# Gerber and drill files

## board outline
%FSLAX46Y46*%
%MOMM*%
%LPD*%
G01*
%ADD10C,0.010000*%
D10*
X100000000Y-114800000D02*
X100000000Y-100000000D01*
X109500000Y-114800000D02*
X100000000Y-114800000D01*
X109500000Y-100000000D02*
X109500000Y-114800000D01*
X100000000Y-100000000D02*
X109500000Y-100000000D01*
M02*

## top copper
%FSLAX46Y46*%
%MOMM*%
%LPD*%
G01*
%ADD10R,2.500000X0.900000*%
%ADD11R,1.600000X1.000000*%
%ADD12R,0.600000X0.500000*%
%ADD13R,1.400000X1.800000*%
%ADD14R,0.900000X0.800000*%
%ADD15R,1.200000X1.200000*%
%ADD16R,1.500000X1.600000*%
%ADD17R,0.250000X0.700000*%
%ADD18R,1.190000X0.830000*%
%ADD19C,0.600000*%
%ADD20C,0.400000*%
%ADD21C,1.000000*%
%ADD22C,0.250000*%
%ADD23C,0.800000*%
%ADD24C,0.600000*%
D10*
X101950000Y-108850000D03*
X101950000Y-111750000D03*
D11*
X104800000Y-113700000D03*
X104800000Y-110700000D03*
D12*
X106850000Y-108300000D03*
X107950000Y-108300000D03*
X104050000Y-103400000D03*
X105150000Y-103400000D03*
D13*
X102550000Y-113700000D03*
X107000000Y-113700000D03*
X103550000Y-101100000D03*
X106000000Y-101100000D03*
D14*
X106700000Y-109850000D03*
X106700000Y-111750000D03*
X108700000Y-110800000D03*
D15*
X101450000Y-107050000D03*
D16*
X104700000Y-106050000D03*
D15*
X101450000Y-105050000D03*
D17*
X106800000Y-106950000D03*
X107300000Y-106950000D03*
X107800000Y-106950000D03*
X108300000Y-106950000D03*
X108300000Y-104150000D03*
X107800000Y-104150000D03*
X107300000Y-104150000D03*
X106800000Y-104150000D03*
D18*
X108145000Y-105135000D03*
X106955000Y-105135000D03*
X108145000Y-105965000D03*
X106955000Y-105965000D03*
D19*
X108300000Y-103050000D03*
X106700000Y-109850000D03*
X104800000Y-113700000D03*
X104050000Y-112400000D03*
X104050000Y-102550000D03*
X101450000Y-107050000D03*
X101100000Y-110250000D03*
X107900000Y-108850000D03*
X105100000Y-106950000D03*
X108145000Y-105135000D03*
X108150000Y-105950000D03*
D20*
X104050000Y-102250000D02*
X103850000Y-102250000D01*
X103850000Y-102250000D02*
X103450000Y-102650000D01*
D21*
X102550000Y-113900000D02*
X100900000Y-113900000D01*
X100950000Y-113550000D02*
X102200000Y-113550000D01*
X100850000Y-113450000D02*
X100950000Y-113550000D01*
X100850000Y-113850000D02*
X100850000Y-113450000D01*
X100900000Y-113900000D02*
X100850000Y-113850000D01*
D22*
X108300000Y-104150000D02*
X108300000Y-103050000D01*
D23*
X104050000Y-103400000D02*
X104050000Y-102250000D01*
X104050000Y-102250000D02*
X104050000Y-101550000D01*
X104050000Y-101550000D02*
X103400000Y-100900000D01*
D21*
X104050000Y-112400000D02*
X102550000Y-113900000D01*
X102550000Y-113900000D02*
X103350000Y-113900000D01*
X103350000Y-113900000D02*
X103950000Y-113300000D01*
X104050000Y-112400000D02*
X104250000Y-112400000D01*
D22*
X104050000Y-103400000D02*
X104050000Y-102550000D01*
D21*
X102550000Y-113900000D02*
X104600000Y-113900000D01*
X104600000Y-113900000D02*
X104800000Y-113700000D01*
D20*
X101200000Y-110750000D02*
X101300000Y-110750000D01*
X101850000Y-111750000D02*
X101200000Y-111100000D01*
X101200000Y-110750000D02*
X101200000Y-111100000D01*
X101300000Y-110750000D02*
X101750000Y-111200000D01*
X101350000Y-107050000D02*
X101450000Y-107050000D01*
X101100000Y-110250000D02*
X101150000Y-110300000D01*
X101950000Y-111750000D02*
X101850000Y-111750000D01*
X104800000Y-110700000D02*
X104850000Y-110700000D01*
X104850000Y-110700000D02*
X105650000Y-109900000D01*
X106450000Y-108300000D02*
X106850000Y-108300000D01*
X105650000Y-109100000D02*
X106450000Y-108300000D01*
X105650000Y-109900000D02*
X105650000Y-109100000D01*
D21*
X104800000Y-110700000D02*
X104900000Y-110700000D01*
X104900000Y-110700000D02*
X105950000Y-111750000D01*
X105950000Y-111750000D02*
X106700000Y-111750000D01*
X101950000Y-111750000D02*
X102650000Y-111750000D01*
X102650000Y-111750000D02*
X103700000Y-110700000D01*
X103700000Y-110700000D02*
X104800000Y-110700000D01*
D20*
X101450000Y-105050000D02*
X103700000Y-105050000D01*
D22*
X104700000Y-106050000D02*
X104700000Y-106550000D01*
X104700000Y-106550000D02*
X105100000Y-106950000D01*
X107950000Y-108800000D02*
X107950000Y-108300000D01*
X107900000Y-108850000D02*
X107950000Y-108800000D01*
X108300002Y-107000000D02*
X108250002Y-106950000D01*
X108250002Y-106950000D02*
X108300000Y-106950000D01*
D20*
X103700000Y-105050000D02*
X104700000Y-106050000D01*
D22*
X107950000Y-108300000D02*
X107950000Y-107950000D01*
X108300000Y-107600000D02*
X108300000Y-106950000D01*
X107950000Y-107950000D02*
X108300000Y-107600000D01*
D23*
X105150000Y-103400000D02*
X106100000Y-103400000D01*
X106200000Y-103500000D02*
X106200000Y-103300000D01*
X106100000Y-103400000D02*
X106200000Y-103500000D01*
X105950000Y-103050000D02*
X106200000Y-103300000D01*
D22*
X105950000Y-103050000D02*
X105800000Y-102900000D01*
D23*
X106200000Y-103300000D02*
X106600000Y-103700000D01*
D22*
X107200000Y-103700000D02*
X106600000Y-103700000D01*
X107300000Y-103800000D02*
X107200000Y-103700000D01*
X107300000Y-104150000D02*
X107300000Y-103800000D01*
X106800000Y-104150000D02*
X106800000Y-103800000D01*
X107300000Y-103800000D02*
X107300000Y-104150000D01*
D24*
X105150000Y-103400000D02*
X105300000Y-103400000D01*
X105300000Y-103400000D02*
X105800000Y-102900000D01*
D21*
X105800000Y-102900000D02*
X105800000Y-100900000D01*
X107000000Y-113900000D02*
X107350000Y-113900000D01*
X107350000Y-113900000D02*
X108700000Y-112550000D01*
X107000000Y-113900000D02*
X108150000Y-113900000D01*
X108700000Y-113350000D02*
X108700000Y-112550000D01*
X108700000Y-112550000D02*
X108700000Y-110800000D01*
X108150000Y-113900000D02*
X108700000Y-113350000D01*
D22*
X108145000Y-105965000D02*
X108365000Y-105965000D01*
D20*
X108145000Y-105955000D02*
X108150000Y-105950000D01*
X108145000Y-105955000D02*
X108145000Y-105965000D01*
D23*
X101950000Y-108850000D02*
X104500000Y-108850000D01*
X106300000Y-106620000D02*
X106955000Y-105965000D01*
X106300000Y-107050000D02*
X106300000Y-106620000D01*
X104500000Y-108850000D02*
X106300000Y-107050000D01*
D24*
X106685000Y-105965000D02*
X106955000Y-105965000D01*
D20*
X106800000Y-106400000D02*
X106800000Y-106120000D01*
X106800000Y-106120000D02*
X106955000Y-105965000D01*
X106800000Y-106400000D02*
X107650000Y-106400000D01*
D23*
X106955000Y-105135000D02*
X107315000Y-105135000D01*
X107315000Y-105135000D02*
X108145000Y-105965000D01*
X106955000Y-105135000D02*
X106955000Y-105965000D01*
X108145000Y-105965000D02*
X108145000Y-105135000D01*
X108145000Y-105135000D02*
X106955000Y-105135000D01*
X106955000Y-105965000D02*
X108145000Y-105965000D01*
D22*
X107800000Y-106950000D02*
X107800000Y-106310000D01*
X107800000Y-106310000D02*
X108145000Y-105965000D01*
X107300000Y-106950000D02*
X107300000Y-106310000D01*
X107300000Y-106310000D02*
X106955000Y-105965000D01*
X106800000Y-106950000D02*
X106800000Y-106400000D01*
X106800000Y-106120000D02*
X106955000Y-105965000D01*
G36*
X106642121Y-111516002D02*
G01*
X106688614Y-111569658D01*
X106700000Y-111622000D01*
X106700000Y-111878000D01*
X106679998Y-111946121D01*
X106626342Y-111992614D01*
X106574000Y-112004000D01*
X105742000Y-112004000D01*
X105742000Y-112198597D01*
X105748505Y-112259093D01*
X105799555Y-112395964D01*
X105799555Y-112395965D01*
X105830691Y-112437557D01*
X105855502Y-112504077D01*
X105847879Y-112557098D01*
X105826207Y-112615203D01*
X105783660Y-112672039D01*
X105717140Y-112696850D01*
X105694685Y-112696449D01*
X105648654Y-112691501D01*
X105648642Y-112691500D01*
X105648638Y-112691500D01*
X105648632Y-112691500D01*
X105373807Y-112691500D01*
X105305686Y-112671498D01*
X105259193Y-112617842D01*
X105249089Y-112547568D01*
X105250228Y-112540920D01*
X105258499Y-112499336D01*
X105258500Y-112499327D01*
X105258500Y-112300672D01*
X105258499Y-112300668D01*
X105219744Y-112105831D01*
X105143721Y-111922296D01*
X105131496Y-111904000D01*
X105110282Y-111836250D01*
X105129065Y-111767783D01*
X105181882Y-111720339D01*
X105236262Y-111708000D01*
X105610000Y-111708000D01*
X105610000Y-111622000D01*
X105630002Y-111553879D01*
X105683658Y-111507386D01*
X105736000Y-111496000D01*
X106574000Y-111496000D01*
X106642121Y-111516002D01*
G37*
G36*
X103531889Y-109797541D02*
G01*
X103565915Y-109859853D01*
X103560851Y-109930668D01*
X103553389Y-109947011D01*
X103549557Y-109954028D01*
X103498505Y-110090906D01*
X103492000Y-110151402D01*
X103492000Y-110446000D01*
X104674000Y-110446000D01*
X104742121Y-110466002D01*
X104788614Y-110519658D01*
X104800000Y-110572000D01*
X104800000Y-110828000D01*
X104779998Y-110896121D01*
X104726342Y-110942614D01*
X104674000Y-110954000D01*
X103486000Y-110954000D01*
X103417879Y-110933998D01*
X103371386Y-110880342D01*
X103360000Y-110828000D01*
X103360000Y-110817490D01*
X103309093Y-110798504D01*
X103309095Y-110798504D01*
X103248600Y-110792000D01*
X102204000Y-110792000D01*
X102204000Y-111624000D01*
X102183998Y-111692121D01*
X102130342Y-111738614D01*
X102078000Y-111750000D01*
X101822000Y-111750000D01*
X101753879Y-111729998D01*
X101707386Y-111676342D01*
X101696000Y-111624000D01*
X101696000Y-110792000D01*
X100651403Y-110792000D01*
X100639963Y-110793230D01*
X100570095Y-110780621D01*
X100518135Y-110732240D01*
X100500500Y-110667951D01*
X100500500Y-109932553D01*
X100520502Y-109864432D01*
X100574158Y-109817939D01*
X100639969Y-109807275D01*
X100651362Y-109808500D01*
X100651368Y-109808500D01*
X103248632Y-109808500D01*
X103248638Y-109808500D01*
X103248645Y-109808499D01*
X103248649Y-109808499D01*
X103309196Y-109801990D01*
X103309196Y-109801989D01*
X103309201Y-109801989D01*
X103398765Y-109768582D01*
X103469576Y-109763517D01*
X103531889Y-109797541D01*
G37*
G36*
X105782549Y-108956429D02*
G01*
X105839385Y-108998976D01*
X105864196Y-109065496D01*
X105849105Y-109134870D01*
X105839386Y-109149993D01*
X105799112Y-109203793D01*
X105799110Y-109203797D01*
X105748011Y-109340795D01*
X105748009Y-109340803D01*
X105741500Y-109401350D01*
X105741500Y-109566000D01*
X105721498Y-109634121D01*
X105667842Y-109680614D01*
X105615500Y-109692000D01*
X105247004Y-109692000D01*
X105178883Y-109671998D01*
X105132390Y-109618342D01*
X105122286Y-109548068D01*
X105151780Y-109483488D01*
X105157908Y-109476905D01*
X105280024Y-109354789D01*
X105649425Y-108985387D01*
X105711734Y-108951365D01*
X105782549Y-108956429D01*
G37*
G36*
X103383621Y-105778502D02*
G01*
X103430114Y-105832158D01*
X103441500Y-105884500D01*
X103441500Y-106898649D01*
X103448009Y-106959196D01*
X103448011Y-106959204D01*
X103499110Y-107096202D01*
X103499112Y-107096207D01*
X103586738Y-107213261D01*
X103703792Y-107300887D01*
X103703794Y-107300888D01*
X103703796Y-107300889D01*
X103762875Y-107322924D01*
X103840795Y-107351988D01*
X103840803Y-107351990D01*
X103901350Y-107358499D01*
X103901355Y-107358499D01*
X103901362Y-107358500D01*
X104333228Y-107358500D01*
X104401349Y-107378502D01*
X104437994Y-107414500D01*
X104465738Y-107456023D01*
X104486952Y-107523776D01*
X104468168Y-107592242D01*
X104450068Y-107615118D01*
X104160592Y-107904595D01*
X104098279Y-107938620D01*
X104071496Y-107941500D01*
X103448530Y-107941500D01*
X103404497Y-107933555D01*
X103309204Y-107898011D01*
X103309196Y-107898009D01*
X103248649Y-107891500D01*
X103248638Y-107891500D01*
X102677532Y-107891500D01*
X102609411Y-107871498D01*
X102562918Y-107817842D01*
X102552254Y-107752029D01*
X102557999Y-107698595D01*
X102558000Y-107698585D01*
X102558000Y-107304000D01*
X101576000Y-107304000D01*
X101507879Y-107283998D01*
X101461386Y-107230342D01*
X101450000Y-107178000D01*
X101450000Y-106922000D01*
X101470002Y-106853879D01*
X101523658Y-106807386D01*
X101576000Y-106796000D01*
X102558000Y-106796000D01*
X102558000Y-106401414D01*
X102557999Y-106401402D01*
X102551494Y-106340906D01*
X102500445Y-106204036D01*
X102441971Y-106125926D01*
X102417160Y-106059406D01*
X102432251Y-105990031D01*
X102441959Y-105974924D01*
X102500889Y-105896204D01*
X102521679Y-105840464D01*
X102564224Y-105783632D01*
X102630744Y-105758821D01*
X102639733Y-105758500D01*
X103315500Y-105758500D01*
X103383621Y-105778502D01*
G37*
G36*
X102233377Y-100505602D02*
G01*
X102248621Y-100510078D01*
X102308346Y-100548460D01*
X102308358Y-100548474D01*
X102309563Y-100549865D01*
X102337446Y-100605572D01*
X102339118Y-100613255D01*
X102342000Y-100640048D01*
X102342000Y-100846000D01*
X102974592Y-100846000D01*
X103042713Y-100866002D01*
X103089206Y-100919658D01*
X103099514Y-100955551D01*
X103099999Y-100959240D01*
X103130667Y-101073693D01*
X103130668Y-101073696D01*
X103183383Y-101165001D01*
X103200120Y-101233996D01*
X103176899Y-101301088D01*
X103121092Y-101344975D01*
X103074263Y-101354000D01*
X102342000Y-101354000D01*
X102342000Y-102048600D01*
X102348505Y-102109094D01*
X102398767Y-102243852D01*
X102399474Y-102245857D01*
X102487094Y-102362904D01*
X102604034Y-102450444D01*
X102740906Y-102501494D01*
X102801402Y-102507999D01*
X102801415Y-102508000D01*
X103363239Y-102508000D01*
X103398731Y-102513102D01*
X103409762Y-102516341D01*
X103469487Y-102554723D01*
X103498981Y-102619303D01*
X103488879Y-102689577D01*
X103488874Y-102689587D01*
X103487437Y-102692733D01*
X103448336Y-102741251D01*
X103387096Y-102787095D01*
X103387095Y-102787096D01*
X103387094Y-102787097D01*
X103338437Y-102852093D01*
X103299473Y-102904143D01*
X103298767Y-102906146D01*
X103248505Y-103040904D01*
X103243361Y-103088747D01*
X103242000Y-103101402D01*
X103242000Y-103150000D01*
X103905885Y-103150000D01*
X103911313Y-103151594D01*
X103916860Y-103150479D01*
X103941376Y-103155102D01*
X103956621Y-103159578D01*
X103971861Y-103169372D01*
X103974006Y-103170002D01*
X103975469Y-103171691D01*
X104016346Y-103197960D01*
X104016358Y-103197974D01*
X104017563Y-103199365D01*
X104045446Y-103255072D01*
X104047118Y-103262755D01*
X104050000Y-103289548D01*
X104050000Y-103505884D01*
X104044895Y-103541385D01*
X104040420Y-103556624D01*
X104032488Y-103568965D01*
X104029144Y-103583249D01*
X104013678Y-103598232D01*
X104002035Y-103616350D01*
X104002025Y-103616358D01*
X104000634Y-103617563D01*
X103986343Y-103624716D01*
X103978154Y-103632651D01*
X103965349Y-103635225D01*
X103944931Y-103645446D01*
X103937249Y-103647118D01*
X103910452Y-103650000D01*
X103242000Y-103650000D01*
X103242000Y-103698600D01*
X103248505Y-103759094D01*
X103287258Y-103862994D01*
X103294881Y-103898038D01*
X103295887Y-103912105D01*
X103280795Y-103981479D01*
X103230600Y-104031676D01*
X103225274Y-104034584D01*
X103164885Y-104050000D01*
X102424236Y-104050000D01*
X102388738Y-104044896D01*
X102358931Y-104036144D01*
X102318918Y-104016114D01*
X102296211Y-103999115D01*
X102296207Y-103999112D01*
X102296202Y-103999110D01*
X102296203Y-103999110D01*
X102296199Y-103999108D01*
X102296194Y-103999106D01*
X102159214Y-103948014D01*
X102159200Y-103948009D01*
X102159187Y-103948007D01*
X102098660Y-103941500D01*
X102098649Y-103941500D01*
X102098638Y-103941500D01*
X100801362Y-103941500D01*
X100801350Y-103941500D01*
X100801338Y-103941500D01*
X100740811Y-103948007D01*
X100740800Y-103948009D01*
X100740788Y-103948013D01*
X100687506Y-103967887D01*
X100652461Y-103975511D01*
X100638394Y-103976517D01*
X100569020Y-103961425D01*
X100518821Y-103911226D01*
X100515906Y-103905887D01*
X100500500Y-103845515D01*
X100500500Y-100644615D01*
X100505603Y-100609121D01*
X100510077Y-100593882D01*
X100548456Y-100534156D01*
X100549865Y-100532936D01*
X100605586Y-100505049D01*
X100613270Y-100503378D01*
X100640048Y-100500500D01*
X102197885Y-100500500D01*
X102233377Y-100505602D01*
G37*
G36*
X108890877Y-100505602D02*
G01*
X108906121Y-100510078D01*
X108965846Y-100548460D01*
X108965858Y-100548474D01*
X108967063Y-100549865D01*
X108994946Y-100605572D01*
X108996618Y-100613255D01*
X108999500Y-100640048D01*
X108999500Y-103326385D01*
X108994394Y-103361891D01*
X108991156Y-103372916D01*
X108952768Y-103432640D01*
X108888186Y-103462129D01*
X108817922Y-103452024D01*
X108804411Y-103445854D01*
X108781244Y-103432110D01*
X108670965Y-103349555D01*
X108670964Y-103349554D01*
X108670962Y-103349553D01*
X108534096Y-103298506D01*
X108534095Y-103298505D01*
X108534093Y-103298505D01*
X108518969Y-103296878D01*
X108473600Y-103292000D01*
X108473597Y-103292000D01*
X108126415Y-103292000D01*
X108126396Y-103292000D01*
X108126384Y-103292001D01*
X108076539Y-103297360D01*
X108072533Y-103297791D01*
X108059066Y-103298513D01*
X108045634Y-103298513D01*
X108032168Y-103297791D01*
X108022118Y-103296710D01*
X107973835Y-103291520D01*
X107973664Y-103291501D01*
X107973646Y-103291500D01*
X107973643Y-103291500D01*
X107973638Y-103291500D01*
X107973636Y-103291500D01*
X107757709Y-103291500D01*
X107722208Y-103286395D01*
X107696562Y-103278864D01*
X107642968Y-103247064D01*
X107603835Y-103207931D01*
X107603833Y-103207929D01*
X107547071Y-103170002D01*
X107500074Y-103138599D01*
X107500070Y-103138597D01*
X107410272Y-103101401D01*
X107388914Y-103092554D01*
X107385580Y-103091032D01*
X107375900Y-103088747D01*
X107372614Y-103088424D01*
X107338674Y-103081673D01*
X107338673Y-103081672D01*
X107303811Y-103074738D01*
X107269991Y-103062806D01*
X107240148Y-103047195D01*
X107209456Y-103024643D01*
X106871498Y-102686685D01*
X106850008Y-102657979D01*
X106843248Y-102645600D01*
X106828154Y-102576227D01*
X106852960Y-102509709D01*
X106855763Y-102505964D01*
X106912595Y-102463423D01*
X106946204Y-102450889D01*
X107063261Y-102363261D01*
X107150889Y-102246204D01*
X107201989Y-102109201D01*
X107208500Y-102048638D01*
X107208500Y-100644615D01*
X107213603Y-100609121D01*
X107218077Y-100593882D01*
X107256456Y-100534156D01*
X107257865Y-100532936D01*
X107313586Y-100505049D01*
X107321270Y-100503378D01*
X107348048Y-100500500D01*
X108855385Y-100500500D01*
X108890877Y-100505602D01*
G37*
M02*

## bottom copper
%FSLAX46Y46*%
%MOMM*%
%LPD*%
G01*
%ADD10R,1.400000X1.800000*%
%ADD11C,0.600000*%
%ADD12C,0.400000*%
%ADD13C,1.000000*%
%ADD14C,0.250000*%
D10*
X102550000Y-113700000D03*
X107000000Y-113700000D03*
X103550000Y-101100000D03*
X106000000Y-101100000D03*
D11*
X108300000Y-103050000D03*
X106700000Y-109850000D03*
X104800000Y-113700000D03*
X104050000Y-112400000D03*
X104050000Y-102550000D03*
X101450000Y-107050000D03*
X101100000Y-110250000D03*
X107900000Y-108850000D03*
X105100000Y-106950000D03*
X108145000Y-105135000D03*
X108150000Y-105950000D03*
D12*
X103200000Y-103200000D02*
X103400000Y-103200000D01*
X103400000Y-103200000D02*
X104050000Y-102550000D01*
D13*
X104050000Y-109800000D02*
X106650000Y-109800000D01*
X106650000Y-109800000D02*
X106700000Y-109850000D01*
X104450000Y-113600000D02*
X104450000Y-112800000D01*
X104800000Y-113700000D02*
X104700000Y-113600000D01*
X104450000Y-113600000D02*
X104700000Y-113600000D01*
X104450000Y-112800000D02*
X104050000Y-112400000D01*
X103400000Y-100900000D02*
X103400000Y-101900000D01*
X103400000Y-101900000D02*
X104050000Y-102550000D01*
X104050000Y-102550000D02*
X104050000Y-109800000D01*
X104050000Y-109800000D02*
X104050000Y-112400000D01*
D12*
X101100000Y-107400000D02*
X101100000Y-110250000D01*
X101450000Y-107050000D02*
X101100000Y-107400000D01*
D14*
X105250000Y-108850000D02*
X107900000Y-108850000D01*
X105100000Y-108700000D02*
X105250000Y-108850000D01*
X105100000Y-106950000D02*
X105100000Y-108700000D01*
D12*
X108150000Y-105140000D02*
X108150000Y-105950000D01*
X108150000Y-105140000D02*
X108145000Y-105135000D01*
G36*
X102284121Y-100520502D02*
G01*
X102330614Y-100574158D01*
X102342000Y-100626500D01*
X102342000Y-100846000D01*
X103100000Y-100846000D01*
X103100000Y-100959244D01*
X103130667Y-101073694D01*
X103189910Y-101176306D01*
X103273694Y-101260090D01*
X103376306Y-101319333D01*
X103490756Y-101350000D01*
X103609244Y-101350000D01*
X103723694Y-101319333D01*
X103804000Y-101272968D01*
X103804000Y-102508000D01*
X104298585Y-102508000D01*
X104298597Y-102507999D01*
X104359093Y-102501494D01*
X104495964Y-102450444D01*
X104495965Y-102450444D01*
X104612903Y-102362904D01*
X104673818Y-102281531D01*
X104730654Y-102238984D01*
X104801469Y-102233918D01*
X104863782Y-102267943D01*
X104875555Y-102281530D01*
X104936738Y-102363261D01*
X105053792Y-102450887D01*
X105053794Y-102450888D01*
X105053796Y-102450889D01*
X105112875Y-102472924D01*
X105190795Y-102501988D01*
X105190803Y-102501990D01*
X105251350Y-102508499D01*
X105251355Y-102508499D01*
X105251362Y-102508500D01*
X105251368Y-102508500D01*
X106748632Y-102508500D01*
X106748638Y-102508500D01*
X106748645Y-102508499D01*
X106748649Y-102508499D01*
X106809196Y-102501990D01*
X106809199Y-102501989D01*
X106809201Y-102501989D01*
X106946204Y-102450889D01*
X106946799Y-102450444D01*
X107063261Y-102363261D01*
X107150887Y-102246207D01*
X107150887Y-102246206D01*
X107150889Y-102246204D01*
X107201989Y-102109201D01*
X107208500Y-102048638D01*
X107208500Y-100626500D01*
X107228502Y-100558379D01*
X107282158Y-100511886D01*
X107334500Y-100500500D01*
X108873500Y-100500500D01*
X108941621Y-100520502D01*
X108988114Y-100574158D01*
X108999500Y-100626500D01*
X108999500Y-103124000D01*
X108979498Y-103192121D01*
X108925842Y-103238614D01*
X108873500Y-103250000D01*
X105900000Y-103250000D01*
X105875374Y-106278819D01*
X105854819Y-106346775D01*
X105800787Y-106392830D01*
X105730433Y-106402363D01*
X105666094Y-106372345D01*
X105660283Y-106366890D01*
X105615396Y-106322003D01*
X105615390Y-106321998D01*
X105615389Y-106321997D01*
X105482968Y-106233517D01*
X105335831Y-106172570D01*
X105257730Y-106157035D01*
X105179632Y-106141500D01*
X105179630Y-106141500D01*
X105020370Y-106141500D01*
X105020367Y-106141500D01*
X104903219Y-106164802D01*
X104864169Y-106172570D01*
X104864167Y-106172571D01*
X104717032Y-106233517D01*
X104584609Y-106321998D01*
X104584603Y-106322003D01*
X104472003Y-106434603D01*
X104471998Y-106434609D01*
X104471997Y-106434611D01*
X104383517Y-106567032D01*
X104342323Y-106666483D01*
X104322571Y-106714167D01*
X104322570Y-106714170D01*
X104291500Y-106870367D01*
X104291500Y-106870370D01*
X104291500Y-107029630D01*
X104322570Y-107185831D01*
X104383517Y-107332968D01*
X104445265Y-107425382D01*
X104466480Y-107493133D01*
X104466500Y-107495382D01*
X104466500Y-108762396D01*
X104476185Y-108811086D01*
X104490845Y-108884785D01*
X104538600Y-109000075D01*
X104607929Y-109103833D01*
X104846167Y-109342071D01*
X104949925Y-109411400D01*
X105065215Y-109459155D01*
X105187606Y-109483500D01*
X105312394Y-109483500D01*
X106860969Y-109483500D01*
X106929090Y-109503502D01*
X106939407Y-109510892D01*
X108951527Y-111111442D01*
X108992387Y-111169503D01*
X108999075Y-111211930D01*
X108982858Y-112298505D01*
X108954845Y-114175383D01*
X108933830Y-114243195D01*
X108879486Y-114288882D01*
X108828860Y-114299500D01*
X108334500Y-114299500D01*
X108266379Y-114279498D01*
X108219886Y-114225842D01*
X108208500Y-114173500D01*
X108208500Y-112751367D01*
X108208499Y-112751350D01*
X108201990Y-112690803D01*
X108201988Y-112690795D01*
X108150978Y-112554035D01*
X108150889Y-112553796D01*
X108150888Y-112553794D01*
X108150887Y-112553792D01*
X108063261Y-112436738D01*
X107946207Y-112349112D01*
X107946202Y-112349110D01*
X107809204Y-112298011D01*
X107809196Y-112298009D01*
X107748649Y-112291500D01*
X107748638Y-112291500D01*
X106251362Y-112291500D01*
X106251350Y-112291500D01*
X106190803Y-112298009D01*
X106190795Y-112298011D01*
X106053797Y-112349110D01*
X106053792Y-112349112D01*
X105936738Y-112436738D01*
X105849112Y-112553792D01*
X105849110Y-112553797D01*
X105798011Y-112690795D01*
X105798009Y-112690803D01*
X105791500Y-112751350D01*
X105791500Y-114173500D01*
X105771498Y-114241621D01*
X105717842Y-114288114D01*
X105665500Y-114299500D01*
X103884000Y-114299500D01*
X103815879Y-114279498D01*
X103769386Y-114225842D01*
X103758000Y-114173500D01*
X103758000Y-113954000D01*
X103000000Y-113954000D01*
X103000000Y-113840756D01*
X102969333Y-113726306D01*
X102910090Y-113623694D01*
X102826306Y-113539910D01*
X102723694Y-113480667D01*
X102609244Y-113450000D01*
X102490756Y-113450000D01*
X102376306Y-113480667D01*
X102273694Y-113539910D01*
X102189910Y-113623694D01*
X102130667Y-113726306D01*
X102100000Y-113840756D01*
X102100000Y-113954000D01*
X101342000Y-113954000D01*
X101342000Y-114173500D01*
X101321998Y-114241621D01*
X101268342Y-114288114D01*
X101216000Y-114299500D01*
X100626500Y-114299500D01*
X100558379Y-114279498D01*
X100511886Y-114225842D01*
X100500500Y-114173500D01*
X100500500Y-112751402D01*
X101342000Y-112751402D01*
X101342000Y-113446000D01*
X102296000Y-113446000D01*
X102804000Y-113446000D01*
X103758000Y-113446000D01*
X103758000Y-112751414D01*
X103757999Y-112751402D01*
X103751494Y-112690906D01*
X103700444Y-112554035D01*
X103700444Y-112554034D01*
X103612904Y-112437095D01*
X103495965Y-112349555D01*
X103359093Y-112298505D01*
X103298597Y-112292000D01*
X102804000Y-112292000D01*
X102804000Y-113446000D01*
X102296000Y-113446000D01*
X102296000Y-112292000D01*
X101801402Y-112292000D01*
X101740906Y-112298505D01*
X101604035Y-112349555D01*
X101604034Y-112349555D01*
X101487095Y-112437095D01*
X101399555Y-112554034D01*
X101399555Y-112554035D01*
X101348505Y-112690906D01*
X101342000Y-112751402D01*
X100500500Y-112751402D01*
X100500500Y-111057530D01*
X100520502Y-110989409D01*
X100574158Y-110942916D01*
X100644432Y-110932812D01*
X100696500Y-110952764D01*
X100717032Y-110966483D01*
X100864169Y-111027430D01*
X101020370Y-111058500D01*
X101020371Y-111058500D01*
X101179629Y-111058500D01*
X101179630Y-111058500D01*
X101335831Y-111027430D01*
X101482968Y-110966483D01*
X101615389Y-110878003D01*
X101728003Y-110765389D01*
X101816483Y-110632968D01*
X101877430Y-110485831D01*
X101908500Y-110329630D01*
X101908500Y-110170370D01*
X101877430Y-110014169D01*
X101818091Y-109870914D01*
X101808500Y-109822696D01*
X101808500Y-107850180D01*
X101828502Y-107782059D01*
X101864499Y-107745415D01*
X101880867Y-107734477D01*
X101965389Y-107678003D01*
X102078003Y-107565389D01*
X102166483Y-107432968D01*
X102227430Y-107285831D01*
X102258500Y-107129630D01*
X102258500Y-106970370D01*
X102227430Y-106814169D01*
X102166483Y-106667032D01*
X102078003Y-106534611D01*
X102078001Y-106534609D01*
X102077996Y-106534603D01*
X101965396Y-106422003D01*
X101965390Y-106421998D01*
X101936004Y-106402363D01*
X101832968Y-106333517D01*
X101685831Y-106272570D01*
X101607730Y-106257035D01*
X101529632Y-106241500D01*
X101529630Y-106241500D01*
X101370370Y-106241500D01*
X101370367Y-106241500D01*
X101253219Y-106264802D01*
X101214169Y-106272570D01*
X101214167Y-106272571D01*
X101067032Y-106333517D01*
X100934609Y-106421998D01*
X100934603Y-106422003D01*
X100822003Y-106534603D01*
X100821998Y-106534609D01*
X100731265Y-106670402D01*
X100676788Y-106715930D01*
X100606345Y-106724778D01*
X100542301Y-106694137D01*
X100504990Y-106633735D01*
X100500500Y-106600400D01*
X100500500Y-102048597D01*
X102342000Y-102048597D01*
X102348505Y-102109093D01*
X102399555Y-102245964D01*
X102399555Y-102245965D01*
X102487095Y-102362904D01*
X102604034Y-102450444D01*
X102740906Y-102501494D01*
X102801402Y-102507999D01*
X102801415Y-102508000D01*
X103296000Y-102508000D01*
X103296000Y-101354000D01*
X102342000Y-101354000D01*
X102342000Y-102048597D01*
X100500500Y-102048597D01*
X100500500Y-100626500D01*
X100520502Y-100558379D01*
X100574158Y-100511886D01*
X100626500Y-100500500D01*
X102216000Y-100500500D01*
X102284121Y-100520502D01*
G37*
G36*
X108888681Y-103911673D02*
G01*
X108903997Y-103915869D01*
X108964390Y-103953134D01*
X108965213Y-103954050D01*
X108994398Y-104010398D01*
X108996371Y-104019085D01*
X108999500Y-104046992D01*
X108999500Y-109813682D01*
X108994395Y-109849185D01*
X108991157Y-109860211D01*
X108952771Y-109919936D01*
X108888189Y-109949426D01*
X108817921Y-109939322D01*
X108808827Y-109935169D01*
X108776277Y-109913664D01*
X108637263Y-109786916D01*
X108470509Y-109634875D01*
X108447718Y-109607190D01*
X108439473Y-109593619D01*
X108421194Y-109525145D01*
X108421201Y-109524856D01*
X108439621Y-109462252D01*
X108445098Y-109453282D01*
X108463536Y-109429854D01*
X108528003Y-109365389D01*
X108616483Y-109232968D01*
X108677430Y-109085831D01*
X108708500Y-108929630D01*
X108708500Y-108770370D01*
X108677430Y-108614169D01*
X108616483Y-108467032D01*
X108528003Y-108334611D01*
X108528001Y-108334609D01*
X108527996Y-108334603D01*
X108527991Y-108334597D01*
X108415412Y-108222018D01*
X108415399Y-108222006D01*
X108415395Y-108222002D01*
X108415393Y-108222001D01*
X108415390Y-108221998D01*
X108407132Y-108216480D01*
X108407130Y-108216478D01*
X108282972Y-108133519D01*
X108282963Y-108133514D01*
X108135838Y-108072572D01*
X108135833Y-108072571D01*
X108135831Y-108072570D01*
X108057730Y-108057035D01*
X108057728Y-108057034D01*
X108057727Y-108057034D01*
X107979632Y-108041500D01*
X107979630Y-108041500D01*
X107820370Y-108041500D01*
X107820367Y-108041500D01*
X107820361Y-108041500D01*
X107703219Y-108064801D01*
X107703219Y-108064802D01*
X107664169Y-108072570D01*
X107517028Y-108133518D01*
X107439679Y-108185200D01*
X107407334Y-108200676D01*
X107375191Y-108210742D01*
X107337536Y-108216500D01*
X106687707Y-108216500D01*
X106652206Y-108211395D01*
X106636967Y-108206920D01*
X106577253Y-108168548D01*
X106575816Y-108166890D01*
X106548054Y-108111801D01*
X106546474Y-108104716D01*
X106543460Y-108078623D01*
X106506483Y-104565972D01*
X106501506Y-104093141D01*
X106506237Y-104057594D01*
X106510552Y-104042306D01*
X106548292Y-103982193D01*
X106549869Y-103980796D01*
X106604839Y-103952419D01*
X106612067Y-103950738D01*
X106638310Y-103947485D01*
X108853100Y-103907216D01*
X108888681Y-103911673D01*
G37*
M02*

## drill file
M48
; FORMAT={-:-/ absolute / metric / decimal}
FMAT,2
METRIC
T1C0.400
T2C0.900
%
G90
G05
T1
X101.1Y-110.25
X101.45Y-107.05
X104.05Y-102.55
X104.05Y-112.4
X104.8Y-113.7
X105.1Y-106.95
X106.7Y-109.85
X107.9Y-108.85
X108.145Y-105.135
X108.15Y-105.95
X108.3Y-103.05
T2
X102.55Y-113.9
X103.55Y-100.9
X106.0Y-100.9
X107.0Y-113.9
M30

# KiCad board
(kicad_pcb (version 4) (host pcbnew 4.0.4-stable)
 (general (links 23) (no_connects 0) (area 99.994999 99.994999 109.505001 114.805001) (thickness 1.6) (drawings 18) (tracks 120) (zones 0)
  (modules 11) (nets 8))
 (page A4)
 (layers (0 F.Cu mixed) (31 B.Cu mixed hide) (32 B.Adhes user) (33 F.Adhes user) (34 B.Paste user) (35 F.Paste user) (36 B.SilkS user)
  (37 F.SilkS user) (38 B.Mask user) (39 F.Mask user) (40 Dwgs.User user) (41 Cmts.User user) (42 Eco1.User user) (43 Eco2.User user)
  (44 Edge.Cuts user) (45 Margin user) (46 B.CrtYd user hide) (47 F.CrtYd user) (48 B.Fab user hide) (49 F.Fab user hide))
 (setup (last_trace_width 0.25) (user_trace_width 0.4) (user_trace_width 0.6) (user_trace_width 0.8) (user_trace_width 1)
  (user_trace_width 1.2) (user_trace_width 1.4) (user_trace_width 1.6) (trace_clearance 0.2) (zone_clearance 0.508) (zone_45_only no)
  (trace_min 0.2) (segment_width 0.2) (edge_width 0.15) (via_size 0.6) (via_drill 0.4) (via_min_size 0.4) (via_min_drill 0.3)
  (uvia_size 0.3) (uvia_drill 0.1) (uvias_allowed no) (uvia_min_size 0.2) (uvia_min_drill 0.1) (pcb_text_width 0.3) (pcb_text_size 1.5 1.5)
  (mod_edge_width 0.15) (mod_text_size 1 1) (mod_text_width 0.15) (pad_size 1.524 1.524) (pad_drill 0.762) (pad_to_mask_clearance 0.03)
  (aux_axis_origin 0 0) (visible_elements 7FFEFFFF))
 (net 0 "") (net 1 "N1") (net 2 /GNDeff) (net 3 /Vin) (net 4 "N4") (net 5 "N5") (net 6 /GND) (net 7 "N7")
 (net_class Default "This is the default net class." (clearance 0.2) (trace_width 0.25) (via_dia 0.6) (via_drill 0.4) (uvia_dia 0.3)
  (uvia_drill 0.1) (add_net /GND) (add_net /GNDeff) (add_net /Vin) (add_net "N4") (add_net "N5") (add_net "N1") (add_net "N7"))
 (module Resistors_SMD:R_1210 (layer F.Cu) (at 101.95 110.3 270)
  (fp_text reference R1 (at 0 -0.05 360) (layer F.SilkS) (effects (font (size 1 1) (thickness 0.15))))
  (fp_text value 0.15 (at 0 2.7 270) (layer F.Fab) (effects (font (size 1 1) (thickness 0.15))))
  (pad 1 smd rect (at -1.45 0 270) (size 0.9 2.5) (layers F.Cu F.Paste F.Mask) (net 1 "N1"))
  (pad 2 smd rect (at 1.45 0 270) (size 0.9 2.5) (layers F.Cu F.Paste F.Mask) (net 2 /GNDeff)))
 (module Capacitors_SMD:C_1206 (layer F.Cu) (at 104.8 112.2 90)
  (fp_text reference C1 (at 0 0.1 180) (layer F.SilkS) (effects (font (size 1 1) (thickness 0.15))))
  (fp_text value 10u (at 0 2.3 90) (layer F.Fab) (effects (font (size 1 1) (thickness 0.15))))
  (pad 1 smd rect (at -1.5 0 90) (size 1 1.6) (layers F.Cu F.Paste F.Mask) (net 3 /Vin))
  (pad 2 smd rect (at 1.5 0 90) (size 1 1.6) (layers F.Cu F.Paste F.Mask) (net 2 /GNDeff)))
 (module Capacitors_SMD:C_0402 (layer F.Cu) (at 107.4 108.3)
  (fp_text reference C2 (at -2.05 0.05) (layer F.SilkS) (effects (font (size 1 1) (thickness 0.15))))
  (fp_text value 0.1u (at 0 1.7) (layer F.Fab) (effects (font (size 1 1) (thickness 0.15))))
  (pad 1 smd rect (at -0.55 0) (size 0.6 0.5) (layers F.Cu F.Paste F.Mask) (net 2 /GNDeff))
  (pad 2 smd rect (at 0.55 0) (size 0.6 0.5) (layers F.Cu F.Paste F.Mask) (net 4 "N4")))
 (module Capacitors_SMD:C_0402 (layer F.Cu) (at 104.6 103.4)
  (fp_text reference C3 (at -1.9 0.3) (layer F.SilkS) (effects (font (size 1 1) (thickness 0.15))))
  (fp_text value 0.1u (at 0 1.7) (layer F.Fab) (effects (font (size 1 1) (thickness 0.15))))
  (pad 1 smd rect (at -0.55 0) (size 0.6 0.5) (layers F.Cu F.Paste F.Mask) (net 3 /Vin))
  (pad 2 smd rect (at 0.55 0) (size 0.6 0.5) (layers F.Cu F.Paste F.Mask) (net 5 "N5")))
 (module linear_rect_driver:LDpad (layer F.Cu) (at 103 113.85 270)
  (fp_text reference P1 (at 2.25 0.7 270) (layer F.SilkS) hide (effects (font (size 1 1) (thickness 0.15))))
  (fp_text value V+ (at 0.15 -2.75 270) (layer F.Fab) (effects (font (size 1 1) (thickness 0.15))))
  (pad 1 thru_hole rect (at 0.05 0.45 270) (size 1.8 1.4) (drill 0.9 (offset -0.2 0)) (layers *.Cu *.Mask) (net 3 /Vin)))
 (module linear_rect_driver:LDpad (layer F.Cu) (at 107.45 113.85 270)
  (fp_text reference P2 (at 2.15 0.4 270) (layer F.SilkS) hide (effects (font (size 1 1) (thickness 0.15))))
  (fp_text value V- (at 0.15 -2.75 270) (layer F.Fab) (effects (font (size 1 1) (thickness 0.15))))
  (pad 1 thru_hole rect (at 0.05 0.45 270) (size 1.8 1.4) (drill 0.9 (offset -0.2 0)) (layers *.Cu *.Mask) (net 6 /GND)))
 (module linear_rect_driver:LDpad (layer F.Cu) (at 103.1 100.95 90)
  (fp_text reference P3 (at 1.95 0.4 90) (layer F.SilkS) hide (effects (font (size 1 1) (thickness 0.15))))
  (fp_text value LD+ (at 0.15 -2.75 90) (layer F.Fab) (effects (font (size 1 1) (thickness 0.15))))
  (pad 1 thru_hole rect (at 0.05 0.45 90) (size 1.8 1.4) (drill 0.9 (offset -0.2 0)) (layers *.Cu *.Mask) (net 3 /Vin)))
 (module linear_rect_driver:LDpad (layer F.Cu) (at 105.55 100.95 90)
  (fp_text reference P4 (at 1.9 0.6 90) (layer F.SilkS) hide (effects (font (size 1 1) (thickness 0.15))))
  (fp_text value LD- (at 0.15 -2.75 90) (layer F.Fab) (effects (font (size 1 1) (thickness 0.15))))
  (pad 1 thru_hole rect (at 0.05 0.45 90) (size 1.8 1.4) (drill 0.9 (offset -0.2 0)) (layers *.Cu *.Mask) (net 5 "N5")))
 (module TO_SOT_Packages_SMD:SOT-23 (layer F.Cu) (at 107.7 110.8)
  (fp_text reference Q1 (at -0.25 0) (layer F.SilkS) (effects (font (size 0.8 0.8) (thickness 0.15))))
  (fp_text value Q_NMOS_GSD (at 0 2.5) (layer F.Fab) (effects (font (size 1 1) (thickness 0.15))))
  (pad 1 smd rect (at -1 -0.95) (size 0.9 0.8) (layers F.Cu F.Paste F.Mask) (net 3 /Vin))
  (pad 2 smd rect (at -1 0.95) (size 0.9 0.8) (layers F.Cu F.Paste F.Mask) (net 2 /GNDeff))
  (pad 3 smd rect (at 1 0) (size 0.9 0.8) (layers F.Cu F.Paste F.Mask) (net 6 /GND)))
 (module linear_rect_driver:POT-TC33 (layer F.Cu) (at 103.95 106.05 270)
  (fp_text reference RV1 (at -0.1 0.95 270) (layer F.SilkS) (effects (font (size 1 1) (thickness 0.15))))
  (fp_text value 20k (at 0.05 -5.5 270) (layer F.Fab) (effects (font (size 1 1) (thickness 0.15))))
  (pad 3 smd rect (at 1 2.5 270) (size 1.2 1.2) (layers F.Cu F.Paste F.Mask) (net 2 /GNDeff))
  (pad 2 smd rect (at 0 -0.75 270) (size 1.6 1.5) (layers F.Cu F.Paste F.Mask) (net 4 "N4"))
  (pad 1 smd rect (at -1 2.5 270) (size 1.2 1.2) (layers F.Cu F.Paste F.Mask) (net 4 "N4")))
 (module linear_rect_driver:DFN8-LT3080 (layer F.Cu) (at 107.55 105.55 90)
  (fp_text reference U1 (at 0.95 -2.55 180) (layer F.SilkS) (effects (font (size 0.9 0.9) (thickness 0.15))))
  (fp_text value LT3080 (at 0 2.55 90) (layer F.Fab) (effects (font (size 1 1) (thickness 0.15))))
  (pad 1 smd rect (at -1.4 -0.75 90) (size 0.7 0.25) (layers F.Cu F.Paste F.Mask) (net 1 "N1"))
  (pad 1 smd rect (at -1.4 -0.25 90) (size 0.7 0.25) (layers F.Cu F.Paste F.Mask) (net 1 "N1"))
  (pad 1 smd rect (at -1.4 0.25 90) (size 0.7 0.25) (layers F.Cu F.Paste F.Mask) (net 1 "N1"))
  (pad 2 smd rect (at -1.4 0.75 90) (size 0.7 0.25) (layers F.Cu F.Paste F.Mask) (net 4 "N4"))
  (pad 3 smd rect (at 1.4 0.75 90) (size 0.7 0.25) (layers F.Cu F.Paste F.Mask) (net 3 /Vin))
  (pad 5 smd rect (at 1.4 0.25 90) (size 0.7 0.25) (layers F.Cu F.Paste F.Mask) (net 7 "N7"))
  (pad 4 smd rect (at 1.4 -0.25 90) (size 0.7 0.25) (layers F.Cu F.Paste F.Mask) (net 5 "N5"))
  (pad 4 smd rect (at 1.4 -0.75 90) (size 0.7 0.25) (layers F.Cu F.Paste F.Mask) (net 5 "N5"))
  (pad 1 smd rect (at 0.415 0.595 90) (size 0.83 1.19) (layers F.Cu F.Paste F.Mask) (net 1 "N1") (solder_paste_margin_ratio -0.2))
  (pad 1 smd rect (at 0.415 -0.595 90) (size 0.83 1.19) (layers F.Cu F.Paste F.Mask) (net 1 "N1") (solder_paste_margin_ratio -0.2))
  (pad 1 smd rect (at -0.415 0.595 90) (size 0.83 1.19) (layers F.Cu F.Paste F.Mask) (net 1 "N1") (solder_paste_margin_ratio -0.2))
  (pad 1 smd rect (at -0.415 -0.595 90) (size 0.83 1.19) (layers F.Cu F.Paste F.Mask) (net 1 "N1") (solder_paste_margin_ratio -0.2)))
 (gr_line (start 100 114.8) (end 100 100) (angle 90) (layer Edge.Cuts) (width 0.01))
 (gr_line (start 109.5 114.8) (end 100 114.8) (angle 90) (layer Edge.Cuts) (width 0.01))
 (gr_line (start 109.5 100) (end 109.5 114.8) (angle 90) (layer Edge.Cuts) (width 0.01))
 (gr_line (start 100 100) (end 109.5 100) (angle 90) (layer Edge.Cuts) (width 0.01))
 (segment (start 104.05 102.25) (end 103.85 102.25) (width 0.4) (layer F.Cu) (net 3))
 (segment (start 103.85 102.25) (end 103.45 102.65) (width 0.4) (layer F.Cu) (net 3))
 (segment (start 103.2 103.2) (end 103.4 103.2) (width 0.4) (layer B.Cu) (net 3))
 (segment (start 103.4 103.2) (end 104.05 102.55) (width 0.4) (layer B.Cu) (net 3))
 (segment (start 102.55 113.9) (end 100.9 113.9) (width 1) (layer F.Cu) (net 3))
 (segment (start 100.95 113.55) (end 102.2 113.55) (width 1) (layer F.Cu) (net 3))
 (segment (start 100.85 113.45) (end 100.95 113.55) (width 1) (layer F.Cu) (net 3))
 (segment (start 100.85 113.85) (end 100.85 113.45) (width 1) (layer F.Cu) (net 3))
 (segment (start 100.9 113.9) (end 100.85 113.85) (width 1) (layer F.Cu) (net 3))
 (segment (start 108.3 104.15) (end 108.3 103.05) (width 0.25) (layer F.Cu) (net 3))
 (via (at 108.3 103.05) (size 0.6) (drill 0.4) (layers F.Cu B.Cu) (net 3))
 (segment (start 104.05 103.4) (end 104.05 102.25) (width 0.8) (layer F.Cu) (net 3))
 (segment (start 104.05 102.25) (end 104.05 101.55) (width 0.8) (layer F.Cu) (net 3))
 (segment (start 104.05 101.55) (end 103.4 100.9) (width 0.8) (layer F.Cu) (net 3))
 (via (at 106.7 109.85) (size 0.6) (drill 0.4) (layers F.Cu B.Cu) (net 3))
 (segment (start 104.05 109.8) (end 106.65 109.8) (width 1) (layer B.Cu) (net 3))
 (segment (start 106.65 109.8) (end 106.7 109.85) (width 1) (layer B.Cu) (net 3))
 (segment (start 104.45 113.6) (end 104.45 112.8) (width 1) (layer B.Cu) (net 3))
 (segment (start 104.8 113.7) (end 104.7 113.6) (width 1) (layer B.Cu) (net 3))
 (segment (start 104.45 113.6) (end 104.7 113.6) (width 1) (layer B.Cu) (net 3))
 (via (at 104.8 113.7) (size 0.6) (drill 0.4) (layers F.Cu B.Cu) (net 3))
 (segment (start 104.45 112.8) (end 104.05 112.4) (width 1) (layer B.Cu) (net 3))
 (segment (start 104.05 112.4) (end 102.55 113.9) (width 1) (layer F.Cu) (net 3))
 (segment (start 102.55 113.9) (end 103.35 113.9) (width 1) (layer F.Cu) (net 3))
 (segment (start 103.35 113.9) (end 103.95 113.3) (width 1) (layer F.Cu) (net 3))
 (via (at 104.05 112.4) (size 0.6) (drill 0.4) (layers F.Cu B.Cu) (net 3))
 (segment (start 104.05 112.4) (end 104.25 112.4) (width 1) (layer F.Cu) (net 3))
 (segment (start 103.4 100.9) (end 103.4 101.9) (width 1) (layer B.Cu) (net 3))
 (segment (start 103.4 101.9) (end 104.05 102.55) (width 1) (layer B.Cu) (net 3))
 (segment (start 104.05 102.55) (end 104.05 109.8) (width 1) (layer B.Cu) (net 3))
 (segment (start 104.05 109.8) (end 104.05 112.4) (width 1) (layer B.Cu) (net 3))
 (via (at 104.05 102.55) (size 0.6) (drill 0.4) (layers F.Cu B.Cu) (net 3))
 (segment (start 104.05 103.4) (end 104.05 102.55) (width 0.25) (layer F.Cu) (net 3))
 (segment (start 102.55 113.9) (end 104.6 113.9) (width 1) (layer F.Cu) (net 3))
 (segment (start 104.6 113.9) (end 104.8 113.7) (width 1) (layer F.Cu) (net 3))
 (segment (start 101.2 110.75) (end 101.3 110.75) (width 0.4) (layer F.Cu) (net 2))
 (segment (start 101.85 111.75) (end 101.2 111.1) (width 0.4) (layer F.Cu) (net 2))
 (segment (start 101.2 110.75) (end 101.2 111.1) (width 0.4) (layer F.Cu) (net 2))
 (segment (start 101.3 110.75) (end 101.75 111.2) (width 0.4) (layer F.Cu) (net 2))
 (via (at 101.45 107.05) (size 0.6) (drill 0.4) (layers F.Cu B.Cu) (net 2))
 (segment (start 101.35 107.05) (end 101.45 107.05) (width 0.4) (layer F.Cu) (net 2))
 (segment (start 101.1 110.25) (end 101.15 110.3) (width 0.4) (layer F.Cu) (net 2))
 (via (at 101.1 110.25) (size 0.6) (drill 0.4) (layers F.Cu B.Cu) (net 2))
 (segment (start 101.1 107.4) (end 101.1 110.25) (width 0.4) (layer B.Cu) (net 2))
 (segment (start 101.45 107.05) (end 101.1 107.4) (width 0.4) (layer B.Cu) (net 2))
 (segment (start 101.95 111.75) (end 101.85 111.75) (width 0.4) (layer F.Cu) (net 2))
 (segment (start 104.8 110.7) (end 104.85 110.7) (width 0.4) (layer F.Cu) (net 2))
 (segment (start 104.85 110.7) (end 105.65 109.9) (width 0.4) (layer F.Cu) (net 2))
 (segment (start 106.45 108.3) (end 106.85 108.3) (width 0.4) (layer F.Cu) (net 2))
 (segment (start 105.65 109.1) (end 106.45 108.3) (width 0.4) (layer F.Cu) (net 2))
 (segment (start 105.65 109.9) (end 105.65 109.1) (width 0.4) (layer F.Cu) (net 2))
 (segment (start 104.8 110.7) (end 104.9 110.7) (width 1) (layer F.Cu) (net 2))
 (segment (start 104.9 110.7) (end 105.95 111.75) (width 1) (layer F.Cu) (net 2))
 (segment (start 105.95 111.75) (end 106.7 111.75) (width 1) (layer F.Cu) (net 2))
 (segment (start 101.95 111.75) (end 102.65 111.75) (width 1) (layer F.Cu) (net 2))
 (segment (start 102.65 111.75) (end 103.7 110.7) (width 1) (layer F.Cu) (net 2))
 (segment (start 103.7 110.7) (end 104.8 110.7) (width 1) (layer F.Cu) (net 2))
 (segment (start 101.45 105.05) (end 103.7 105.05) (width 0.4) (layer F.Cu) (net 4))
 (segment (start 104.7 106.05) (end 104.7 106.55) (width 0.25) (layer F.Cu) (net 4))
 (segment (start 104.7 106.55) (end 105.1 106.95) (width 0.25) (layer F.Cu) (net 4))
 (segment (start 107.95 108.8) (end 107.95 108.3) (width 0.25) (layer F.Cu) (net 4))
 (segment (start 107.9 108.85) (end 107.95 108.8) (width 0.25) (layer F.Cu) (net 4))
 (via (at 107.9 108.85) (size 0.6) (drill 0.4) (layers F.Cu B.Cu) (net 4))
 (segment (start 105.25 108.85) (end 107.9 108.85) (width 0.25) (layer B.Cu) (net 4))
 (segment (start 105.1 108.7) (end 105.25 108.85) (width 0.25) (layer B.Cu) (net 4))
 (segment (start 105.1 106.95) (end 105.1 108.7) (width 0.25) (layer B.Cu) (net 4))
 (via (at 105.1 106.95) (size 0.6) (drill 0.4) (layers F.Cu B.Cu) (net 4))
 (segment (start 108.300002 107) (end 108.250002 106.95) (width 0.25) (layer F.Cu) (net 4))
 (segment (start 108.250002 106.95) (end 108.3 106.95) (width 0.25) (layer F.Cu) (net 4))
 (segment (start 103.7 105.05) (end 104.7 106.05) (width 0.4) (layer F.Cu) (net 4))
 (segment (start 107.95 108.3) (end 107.95 107.95) (width 0.25) (layer F.Cu) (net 4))
 (segment (start 108.3 107.6) (end 108.3 106.95) (width 0.25) (layer F.Cu) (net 4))
 (segment (start 107.95 107.95) (end 108.3 107.6) (width 0.25) (layer F.Cu) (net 4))
 (segment (start 105.15 103.4) (end 106.1 103.4) (width 0.8) (layer F.Cu) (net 5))
 (segment (start 106.2 103.5) (end 106.2 103.3) (width 0.8) (layer F.Cu) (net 5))
 (segment (start 106.1 103.4) (end 106.2 103.5) (width 0.8) (layer F.Cu) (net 5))
 (segment (start 105.95 103.05) (end 106.2 103.3) (width 0.8) (layer F.Cu) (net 5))
 (segment (start 105.95 103.05) (end 105.8 102.9) (width 0.25) (layer F.Cu) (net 5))
 (segment (start 106.2 103.3) (end 106.6 103.7) (width 0.8) (layer F.Cu) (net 5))
 (segment (start 107.2 103.7) (end 106.6 103.7) (width 0.25) (layer F.Cu) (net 5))
 (segment (start 107.3 103.8) (end 107.2 103.7) (width 0.25) (layer F.Cu) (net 5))
 (segment (start 107.3 104.15) (end 107.3 103.8) (width 0.25) (layer F.Cu) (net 5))
 (segment (start 106.8 104.15) (end 106.8 103.8) (width 0.25) (layer F.Cu) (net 5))
 (segment (start 107.3 103.8) (end 107.3 104.15) (width 0.25) (layer F.Cu) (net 5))
 (segment (start 105.15 103.4) (end 105.3 103.4) (width 0.6) (layer F.Cu) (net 5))
 (segment (start 105.3 103.4) (end 105.8 102.9) (width 0.6) (layer F.Cu) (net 5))
 (segment (start 105.8 102.9) (end 105.8 100.9) (width 1) (layer F.Cu) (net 5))
 (segment (start 107 113.9) (end 107.35 113.9) (width 1) (layer F.Cu) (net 6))
 (segment (start 107.35 113.9) (end 108.7 112.55) (width 1) (layer F.Cu) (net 6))
 (segment (start 107 113.9) (end 108.15 113.9) (width 1) (layer F.Cu) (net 6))
 (segment (start 108.7 113.35) (end 108.7 112.55) (width 1) (layer F.Cu) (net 6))
 (segment (start 108.7 112.55) (end 108.7 110.8) (width 1) (layer F.Cu) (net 6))
 (segment (start 108.15 113.9) (end 108.7 113.35) (width 1) (layer F.Cu) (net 6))
 (segment (start 108.145 105.965) (end 108.365 105.965) (width 0.25) (layer F.Cu) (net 1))
 (via (at 108.145 105.135) (size 0.6) (drill 0.4) (layers F.Cu B.Cu) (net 1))
 (segment (start 108.145 105.955) (end 108.15 105.95) (width 0.4) (layer F.Cu) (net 1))
 (via (at 108.15 105.95) (size 0.6) (drill 0.4) (layers F.Cu B.Cu) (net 1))
 (segment (start 108.15 105.14) (end 108.15 105.95) (width 0.4) (layer B.Cu) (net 1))
 (segment (start 108.15 105.14) (end 108.145 105.135) (width 0.4) (layer B.Cu) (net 1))
 (segment (start 108.145 105.955) (end 108.145 105.965) (width 0.4) (layer F.Cu) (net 1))
 (segment (start 101.95 108.85) (end 104.5 108.85) (width 0.8) (layer F.Cu) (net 1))
 (segment (start 106.3 106.62) (end 106.955 105.965) (width 0.8) (layer F.Cu) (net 1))
 (segment (start 106.3 107.05) (end 106.3 106.62) (width 0.8) (layer F.Cu) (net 1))
 (segment (start 104.5 108.85) (end 106.3 107.05) (width 0.8) (layer F.Cu) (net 1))
 (segment (start 106.685 105.965) (end 106.955 105.965) (width 0.6) (layer F.Cu) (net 1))
 (segment (start 106.8 106.4) (end 106.8 106.12) (width 0.4) (layer F.Cu) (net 1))
 (segment (start 106.8 106.12) (end 106.955 105.965) (width 0.4) (layer F.Cu) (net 1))
 (segment (start 106.8 106.4) (end 107.65 106.4) (width 0.4) (layer F.Cu) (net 1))
 (segment (start 106.955 105.135) (end 107.315 105.135) (width 0.8) (layer F.Cu) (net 1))
 (segment (start 107.315 105.135) (end 108.145 105.965) (width 0.8) (layer F.Cu) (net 1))
 (segment (start 106.955 105.135) (end 106.955 105.965) (width 0.8) (layer F.Cu) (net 1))
 (segment (start 108.145 105.965) (end 108.145 105.135) (width 0.8) (layer F.Cu) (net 1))
 (segment (start 108.145 105.135) (end 106.955 105.135) (width 0.8) (layer F.Cu) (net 1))
 (segment (start 106.955 105.965) (end 108.145 105.965) (width 0.8) (layer F.Cu) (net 1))
 (segment (start 107.8 106.95) (end 107.8 106.31) (width 0.25) (layer F.Cu) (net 1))
 (segment (start 107.8 106.31) (end 108.145 105.965) (width 0.25) (layer F.Cu) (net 1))
 (segment (start 107.3 106.95) (end 107.3 106.31) (width 0.25) (layer F.Cu) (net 1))
 (segment (start 107.3 106.31) (end 106.955 105.965) (width 0.25) (layer F.Cu) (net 1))
 (segment (start 106.8 106.95) (end 106.8 106.4) (width 0.25) (layer F.Cu) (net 1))
 (segment (start 106.8 106.12) (end 106.955 105.965) (width 0.25) (layer F.Cu) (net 1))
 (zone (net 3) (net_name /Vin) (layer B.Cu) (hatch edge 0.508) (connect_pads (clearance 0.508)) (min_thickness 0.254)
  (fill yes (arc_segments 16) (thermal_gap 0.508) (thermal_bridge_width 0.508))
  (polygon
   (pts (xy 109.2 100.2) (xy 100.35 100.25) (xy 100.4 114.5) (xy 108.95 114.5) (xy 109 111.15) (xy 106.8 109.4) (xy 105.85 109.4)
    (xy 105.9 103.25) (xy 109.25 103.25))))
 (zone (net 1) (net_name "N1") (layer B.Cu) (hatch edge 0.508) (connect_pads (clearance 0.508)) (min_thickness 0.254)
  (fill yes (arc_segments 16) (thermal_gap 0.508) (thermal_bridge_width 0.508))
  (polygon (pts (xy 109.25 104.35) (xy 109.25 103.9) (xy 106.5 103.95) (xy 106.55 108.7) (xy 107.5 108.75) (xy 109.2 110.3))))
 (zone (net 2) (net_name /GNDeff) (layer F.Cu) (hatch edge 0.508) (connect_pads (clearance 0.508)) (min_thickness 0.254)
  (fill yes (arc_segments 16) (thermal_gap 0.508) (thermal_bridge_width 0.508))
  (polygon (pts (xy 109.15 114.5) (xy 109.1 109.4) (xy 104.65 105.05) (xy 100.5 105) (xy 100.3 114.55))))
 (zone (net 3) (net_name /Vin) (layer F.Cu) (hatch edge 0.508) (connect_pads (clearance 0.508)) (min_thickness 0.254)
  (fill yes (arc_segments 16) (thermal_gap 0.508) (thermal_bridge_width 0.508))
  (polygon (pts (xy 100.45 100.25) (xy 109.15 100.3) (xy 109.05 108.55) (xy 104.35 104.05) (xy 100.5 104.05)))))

